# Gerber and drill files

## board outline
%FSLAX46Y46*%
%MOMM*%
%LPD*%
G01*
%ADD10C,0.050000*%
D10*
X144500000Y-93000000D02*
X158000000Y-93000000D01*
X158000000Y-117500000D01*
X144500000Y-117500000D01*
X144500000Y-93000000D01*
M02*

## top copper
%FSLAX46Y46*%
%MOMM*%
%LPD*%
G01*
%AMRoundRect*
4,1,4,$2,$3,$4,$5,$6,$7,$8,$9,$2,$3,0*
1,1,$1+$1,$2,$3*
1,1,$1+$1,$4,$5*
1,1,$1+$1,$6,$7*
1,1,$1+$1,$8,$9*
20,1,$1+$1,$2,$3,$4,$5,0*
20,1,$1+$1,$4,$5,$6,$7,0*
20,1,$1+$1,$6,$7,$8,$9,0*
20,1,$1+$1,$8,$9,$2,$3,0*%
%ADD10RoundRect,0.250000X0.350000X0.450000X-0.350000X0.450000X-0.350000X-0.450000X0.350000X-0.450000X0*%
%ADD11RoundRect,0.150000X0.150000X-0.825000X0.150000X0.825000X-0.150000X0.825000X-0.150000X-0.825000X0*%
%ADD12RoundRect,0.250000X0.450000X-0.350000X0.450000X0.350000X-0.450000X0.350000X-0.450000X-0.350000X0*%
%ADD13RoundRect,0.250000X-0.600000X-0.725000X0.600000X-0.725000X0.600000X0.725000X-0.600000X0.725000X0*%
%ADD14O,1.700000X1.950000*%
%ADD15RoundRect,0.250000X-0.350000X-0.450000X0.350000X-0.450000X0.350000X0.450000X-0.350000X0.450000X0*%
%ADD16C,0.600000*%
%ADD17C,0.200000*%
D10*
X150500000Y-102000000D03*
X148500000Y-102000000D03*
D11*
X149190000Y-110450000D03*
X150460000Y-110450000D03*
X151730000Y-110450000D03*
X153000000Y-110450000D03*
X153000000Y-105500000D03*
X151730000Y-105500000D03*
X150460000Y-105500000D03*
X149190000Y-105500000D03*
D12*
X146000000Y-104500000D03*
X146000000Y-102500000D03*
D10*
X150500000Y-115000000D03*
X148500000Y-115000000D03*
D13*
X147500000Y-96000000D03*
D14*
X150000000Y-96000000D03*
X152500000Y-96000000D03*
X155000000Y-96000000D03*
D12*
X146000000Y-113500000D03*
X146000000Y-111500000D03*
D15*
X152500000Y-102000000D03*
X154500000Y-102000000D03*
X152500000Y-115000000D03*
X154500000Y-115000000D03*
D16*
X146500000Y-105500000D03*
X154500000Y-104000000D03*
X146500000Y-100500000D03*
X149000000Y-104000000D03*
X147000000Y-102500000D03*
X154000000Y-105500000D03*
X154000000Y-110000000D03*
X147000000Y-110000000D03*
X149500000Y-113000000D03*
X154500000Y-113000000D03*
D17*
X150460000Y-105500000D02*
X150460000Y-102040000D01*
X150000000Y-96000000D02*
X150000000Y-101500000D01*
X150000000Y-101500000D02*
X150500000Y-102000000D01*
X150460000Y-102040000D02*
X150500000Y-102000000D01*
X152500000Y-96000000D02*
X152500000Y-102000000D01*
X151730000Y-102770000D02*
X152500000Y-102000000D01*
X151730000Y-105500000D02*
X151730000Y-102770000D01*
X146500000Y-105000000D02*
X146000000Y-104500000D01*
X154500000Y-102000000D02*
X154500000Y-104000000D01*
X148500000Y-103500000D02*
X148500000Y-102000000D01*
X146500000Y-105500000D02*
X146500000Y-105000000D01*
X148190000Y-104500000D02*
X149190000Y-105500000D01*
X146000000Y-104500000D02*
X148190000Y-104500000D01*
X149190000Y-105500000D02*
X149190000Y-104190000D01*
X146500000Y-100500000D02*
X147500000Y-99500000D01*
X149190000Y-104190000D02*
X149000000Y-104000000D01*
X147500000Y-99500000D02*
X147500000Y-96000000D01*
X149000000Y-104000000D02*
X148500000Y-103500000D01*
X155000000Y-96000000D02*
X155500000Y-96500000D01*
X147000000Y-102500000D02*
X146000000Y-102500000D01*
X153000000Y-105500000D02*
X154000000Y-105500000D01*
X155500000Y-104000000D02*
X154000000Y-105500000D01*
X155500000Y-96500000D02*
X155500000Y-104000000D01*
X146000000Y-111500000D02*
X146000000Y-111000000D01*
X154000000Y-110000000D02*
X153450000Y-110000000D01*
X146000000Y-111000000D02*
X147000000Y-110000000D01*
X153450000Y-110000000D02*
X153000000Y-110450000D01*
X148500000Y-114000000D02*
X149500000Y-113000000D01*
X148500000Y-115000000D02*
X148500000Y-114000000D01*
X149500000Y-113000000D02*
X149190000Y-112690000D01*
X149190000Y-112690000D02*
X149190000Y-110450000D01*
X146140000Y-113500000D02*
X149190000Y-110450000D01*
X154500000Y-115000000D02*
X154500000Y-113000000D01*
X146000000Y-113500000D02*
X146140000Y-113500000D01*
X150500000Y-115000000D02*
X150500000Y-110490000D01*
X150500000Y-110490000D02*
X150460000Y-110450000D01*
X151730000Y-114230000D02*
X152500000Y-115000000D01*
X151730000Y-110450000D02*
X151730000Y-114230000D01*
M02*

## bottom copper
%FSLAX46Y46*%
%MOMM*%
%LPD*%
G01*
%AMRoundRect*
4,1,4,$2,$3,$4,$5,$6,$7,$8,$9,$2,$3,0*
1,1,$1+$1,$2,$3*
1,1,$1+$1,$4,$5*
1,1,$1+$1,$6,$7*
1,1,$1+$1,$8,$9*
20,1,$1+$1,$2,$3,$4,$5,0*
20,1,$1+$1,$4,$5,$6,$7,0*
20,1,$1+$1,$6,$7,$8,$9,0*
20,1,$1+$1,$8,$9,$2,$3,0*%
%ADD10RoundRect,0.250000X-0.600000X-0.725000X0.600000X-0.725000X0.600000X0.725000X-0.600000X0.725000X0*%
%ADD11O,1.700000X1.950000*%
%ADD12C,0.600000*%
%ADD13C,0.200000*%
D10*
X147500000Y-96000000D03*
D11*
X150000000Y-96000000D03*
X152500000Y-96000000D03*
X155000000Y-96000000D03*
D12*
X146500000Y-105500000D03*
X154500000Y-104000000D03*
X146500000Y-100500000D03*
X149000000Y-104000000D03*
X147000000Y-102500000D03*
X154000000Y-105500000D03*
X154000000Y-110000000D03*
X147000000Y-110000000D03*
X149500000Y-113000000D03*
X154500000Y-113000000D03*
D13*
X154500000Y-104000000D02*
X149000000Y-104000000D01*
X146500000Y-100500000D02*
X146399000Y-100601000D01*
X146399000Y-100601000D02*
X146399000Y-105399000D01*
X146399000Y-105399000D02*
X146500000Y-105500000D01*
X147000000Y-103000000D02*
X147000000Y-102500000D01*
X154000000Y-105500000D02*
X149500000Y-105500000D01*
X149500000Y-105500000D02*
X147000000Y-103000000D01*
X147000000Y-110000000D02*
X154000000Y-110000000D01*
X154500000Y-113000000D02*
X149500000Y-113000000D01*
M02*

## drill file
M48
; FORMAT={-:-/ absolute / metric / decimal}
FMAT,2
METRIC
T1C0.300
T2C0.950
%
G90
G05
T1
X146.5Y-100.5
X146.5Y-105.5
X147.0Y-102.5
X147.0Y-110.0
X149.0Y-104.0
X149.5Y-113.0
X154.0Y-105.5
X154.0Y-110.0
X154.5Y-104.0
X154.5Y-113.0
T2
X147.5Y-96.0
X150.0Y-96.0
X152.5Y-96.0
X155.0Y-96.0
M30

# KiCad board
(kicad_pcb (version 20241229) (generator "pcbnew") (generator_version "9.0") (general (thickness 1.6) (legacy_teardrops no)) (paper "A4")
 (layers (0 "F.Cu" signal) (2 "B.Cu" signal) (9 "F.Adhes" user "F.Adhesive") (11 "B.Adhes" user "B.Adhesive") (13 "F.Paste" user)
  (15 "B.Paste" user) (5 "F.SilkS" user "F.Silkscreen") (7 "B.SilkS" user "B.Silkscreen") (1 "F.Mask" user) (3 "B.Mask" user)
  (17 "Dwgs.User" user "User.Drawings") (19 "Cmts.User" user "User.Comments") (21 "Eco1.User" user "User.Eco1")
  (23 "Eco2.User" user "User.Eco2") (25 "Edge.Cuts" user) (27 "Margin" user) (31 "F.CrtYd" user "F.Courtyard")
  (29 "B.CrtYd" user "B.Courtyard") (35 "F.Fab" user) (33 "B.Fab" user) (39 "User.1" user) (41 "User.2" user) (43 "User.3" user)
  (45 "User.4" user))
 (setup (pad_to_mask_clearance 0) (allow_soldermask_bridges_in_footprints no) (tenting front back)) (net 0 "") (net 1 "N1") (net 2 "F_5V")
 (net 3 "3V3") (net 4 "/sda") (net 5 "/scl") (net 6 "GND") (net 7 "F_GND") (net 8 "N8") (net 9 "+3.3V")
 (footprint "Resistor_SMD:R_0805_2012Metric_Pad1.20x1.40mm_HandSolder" (layer "F.Cu") (at 149.5 102 180)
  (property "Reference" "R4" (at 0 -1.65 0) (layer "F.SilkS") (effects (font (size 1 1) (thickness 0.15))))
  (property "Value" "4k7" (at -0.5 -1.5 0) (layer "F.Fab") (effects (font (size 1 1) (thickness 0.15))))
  (pad "1" smd roundrect (at -1 0 180) (size 1.2 1.4) (layers "F.Cu" "F.Mask" "F.Paste") (roundrect_rratio 0.208333) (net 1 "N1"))
  (pad "2" smd roundrect (at 1 0 180) (size 1.2 1.4) (layers "F.Cu" "F.Mask" "F.Paste") (roundrect_rratio 0.208333) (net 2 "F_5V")))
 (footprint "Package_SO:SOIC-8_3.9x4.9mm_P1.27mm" (layer "F.Cu") (at 151.095 107.975 90)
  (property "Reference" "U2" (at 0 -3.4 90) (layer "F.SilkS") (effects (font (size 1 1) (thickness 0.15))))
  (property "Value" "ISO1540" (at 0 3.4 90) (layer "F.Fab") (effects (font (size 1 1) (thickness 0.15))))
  (pad "1" smd roundrect (at -2.475 -1.905 90) (size 1.95 0.6) (layers "F.Cu" "F.Mask" "F.Paste") (roundrect_rratio 0.25) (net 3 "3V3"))
  (pad "2" smd roundrect (at -2.475 -0.635 90) (size 1.95 0.6) (layers "F.Cu" "F.Mask" "F.Paste") (roundrect_rratio 0.25) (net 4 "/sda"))
  (pad "3" smd roundrect (at -2.475 0.635 90) (size 1.95 0.6) (layers "F.Cu" "F.Mask" "F.Paste") (roundrect_rratio 0.25) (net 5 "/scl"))
  (pad "4" smd roundrect (at -2.475 1.905 90) (size 1.95 0.6) (layers "F.Cu" "F.Mask" "F.Paste") (roundrect_rratio 0.25) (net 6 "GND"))
  (pad "5" smd roundrect (at 2.475 1.905 90) (size 1.95 0.6) (layers "F.Cu" "F.Mask" "F.Paste") (roundrect_rratio 0.25) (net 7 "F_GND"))
  (pad "6" smd roundrect (at 2.475 0.635 90) (size 1.95 0.6) (layers "F.Cu" "F.Mask" "F.Paste") (roundrect_rratio 0.25) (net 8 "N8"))
  (pad "7" smd roundrect (at 2.475 -0.635 90) (size 1.95 0.6) (layers "F.Cu" "F.Mask" "F.Paste") (roundrect_rratio 0.25) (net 1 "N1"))
  (pad "8" smd roundrect (at 2.475 -1.905 90) (size 1.95 0.6) (layers "F.Cu" "F.Mask" "F.Paste") (roundrect_rratio 0.25) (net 2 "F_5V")))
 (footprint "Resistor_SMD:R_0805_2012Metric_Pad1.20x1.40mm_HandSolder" (layer "F.Cu") (at 146 103.5 90)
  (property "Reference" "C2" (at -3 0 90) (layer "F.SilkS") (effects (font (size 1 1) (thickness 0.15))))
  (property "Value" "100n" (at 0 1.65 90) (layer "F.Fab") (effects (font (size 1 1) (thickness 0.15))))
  (pad "1" smd roundrect (at -1 0 90) (size 1.2 1.4) (layers "F.Cu" "F.Mask" "F.Paste") (roundrect_rratio 0.208333) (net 2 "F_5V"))
  (pad "2" smd roundrect (at 1 0 90) (size 1.2 1.4) (layers "F.Cu" "F.Mask" "F.Paste") (roundrect_rratio 0.208333) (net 7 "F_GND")))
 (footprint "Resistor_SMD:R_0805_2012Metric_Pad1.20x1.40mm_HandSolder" (layer "F.Cu") (at 149.5 115 180)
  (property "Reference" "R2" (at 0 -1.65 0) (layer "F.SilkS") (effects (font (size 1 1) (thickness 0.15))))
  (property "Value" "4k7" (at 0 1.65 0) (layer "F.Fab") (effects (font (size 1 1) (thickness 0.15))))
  (pad "1" smd roundrect (at -1 0 180) (size 1.2 1.4) (layers "F.Cu" "F.Mask" "F.Paste") (roundrect_rratio 0.208333) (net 4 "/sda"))
  (pad "2" smd roundrect (at 1 0 180) (size 1.2 1.4) (layers "F.Cu" "F.Mask" "F.Paste") (roundrect_rratio 0.208333) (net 3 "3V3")))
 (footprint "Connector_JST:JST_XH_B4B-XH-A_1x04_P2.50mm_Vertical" (layer "F.Cu") (at 147.5 96)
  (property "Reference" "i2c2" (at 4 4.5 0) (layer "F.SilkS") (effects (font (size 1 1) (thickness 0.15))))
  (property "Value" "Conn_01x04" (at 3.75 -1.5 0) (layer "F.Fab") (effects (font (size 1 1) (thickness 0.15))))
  (pad "1" thru_hole roundrect (at 0 0) (size 1.7 1.95) (drill 0.95) (layers "*.Cu" "*.Mask") (remove_unused_layers no)
   (roundrect_rratio 0.147059) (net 2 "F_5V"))
  (pad "2" thru_hole oval (at 2.5 0) (size 1.7 1.95) (drill 0.95) (layers "*.Cu" "*.Mask") (remove_unused_layers no) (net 1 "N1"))
  (pad "3" thru_hole oval (at 5 0) (size 1.7 1.95) (drill 0.95) (layers "*.Cu" "*.Mask") (remove_unused_layers no) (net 8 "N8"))
  (pad "4" thru_hole oval (at 7.5 0) (size 1.7 1.95) (drill 0.95) (layers "*.Cu" "*.Mask") (remove_unused_layers no) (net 7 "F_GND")))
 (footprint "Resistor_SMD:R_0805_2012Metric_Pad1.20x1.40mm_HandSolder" (layer "F.Cu") (at 146 112.5 90)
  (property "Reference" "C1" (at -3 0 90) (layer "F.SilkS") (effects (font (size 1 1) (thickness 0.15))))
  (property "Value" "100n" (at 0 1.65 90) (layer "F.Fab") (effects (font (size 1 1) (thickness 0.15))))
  (pad "1" smd roundrect (at -1 0 90) (size 1.2 1.4) (layers "F.Cu" "F.Mask" "F.Paste") (roundrect_rratio 0.208333) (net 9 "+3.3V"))
  (pad "2" smd roundrect (at 1 0 90) (size 1.2 1.4) (layers "F.Cu" "F.Mask" "F.Paste") (roundrect_rratio 0.208333) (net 6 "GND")))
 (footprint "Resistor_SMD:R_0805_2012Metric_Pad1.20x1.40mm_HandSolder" (layer "F.Cu") (at 153.5 102)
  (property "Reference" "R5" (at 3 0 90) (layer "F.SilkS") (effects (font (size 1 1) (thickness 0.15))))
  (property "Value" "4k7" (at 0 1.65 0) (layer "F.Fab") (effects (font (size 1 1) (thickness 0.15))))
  (pad "1" smd roundrect (at -1 0) (size 1.2 1.4) (layers "F.Cu" "F.Mask" "F.Paste") (roundrect_rratio 0.208333) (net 8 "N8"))
  (pad "2" smd roundrect (at 1 0) (size 1.2 1.4) (layers "F.Cu" "F.Mask" "F.Paste") (roundrect_rratio 0.208333) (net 2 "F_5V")))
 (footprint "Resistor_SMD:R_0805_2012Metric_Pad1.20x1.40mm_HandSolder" (layer "F.Cu") (at 153.5 115)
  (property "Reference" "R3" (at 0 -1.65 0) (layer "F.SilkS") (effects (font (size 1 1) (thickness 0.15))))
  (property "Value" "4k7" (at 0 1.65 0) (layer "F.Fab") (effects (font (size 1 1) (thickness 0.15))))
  (pad "1" smd roundrect (at -1 0) (size 1.2 1.4) (layers "F.Cu" "F.Mask" "F.Paste") (roundrect_rratio 0.208333) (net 5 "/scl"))
  (pad "2" smd roundrect (at 1 0) (size 1.2 1.4) (layers "F.Cu" "F.Mask" "F.Paste") (roundrect_rratio 0.208333) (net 3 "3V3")))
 (gr_rect (start 144.5 93) (end 158 117.5) (stroke (width 0.05) (type default)) (fill no) (layer "Edge.Cuts"))
 (segment (start 150.46 105.5) (end 150.46 102.04) (width 0.2) (layer "F.Cu") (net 1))
 (segment (start 150 96) (end 150 101.5) (width 0.2) (layer "F.Cu") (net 1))
 (segment (start 150 101.5) (end 150.5 102) (width 0.2) (layer "F.Cu") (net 1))
 (segment (start 150.46 102.04) (end 150.5 102) (width 0.2) (layer "F.Cu") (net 1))
 (segment (start 152.5 96) (end 152.5 102) (width 0.2) (layer "F.Cu") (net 8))
 (segment (start 151.73 102.77) (end 152.5 102) (width 0.2) (layer "F.Cu") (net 8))
 (segment (start 151.73 105.5) (end 151.73 102.77) (width 0.2) (layer "F.Cu") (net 8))
 (segment (start 146.5 105) (end 146 104.5) (width 0.2) (layer "F.Cu") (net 2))
 (segment (start 154.5 102) (end 154.5 104) (width 0.2) (layer "F.Cu") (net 2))
 (segment (start 148.5 103.5) (end 148.5 102) (width 0.2) (layer "F.Cu") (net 2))
 (segment (start 146.5 105.5) (end 146.5 105) (width 0.2) (layer "F.Cu") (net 2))
 (segment (start 148.19 104.5) (end 149.19 105.5) (width 0.2) (layer "F.Cu") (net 2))
 (segment (start 146 104.5) (end 148.19 104.5) (width 0.2) (layer "F.Cu") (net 2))
 (segment (start 149.19 105.5) (end 149.19 104.19) (width 0.2) (layer "F.Cu") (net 2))
 (segment (start 146.5 100.5) (end 147.5 99.5) (width 0.2) (layer "F.Cu") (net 2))
 (segment (start 149.19 104.19) (end 149 104) (width 0.2) (layer "F.Cu") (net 2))
 (segment (start 147.5 99.5) (end 147.5 96) (width 0.2) (layer "F.Cu") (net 2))
 (segment (start 149 104) (end 148.5 103.5) (width 0.2) (layer "F.Cu") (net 2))
 (via (at 146.5 105.5) (size 0.6) (drill 0.3) (layers "F.Cu" "B.Cu") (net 2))
 (via (at 154.5 104) (size 0.6) (drill 0.3) (layers "F.Cu" "B.Cu") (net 2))
 (via (at 146.5 100.5) (size 0.6) (drill 0.3) (layers "F.Cu" "B.Cu") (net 2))
 (via (at 149 104) (size 0.6) (drill 0.3) (layers "F.Cu" "B.Cu") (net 2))
 (segment (start 154.5 104) (end 149 104) (width 0.2) (layer "B.Cu") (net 2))
 (segment (start 146.5 100.5) (end 146.399 100.601) (width 0.2) (layer "B.Cu") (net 2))
 (segment (start 146.399 100.601) (end 146.399 105.399) (width 0.2) (layer "B.Cu") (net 2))
 (segment (start 146.399 105.399) (end 146.5 105.5) (width 0.2) (layer "B.Cu") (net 2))
 (segment (start 155 96) (end 155.5 96.5) (width 0.2) (layer "F.Cu") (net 7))
 (segment (start 147 102.5) (end 146 102.5) (width 0.2) (layer "F.Cu") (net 7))
 (segment (start 153 105.5) (end 154 105.5) (width 0.2) (layer "F.Cu") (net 7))
 (segment (start 155.5 104) (end 154 105.5) (width 0.2) (layer "F.Cu") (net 7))
 (segment (start 155.5 96.5) (end 155.5 104) (width 0.2) (layer "F.Cu") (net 7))
 (via (at 147 102.5) (size 0.6) (drill 0.3) (layers "F.Cu" "B.Cu") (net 7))
 (via (at 154 105.5) (size 0.6) (drill 0.3) (layers "F.Cu" "B.Cu") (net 7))
 (segment (start 147 103) (end 147 102.5) (width 0.2) (layer "B.Cu") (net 7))
 (segment (start 154 105.5) (end 149.5 105.5) (width 0.2) (layer "B.Cu") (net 7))
 (segment (start 149.5 105.5) (end 147 103) (width 0.2) (layer "B.Cu") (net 7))
 (segment (start 146 111.5) (end 146 111) (width 0.2) (layer "F.Cu") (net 6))
 (segment (start 154 110) (end 153.45 110) (width 0.2) (layer "F.Cu") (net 6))
 (segment (start 146 111) (end 147 110) (width 0.2) (layer "F.Cu") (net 6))
 (segment (start 153.45 110) (end 153 110.45) (width 0.2) (layer "F.Cu") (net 6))
 (via (at 154 110) (size 0.6) (drill 0.3) (layers "F.Cu" "B.Cu") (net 6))
 (via (at 147 110) (size 0.6) (drill 0.3) (layers "F.Cu" "B.Cu") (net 6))
 (segment (start 147 110) (end 154 110) (width 0.2) (layer "B.Cu") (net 6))
 (segment (start 148.5 114) (end 149.5 113) (width 0.2) (layer "F.Cu") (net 9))
 (segment (start 148.5 115) (end 148.5 114) (width 0.2) (layer "F.Cu") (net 9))
 (segment (start 149.5 113) (end 149.19 112.69) (width 0.2) (layer "F.Cu") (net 9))
 (segment (start 149.19 112.69) (end 149.19 110.45) (width 0.2) (layer "F.Cu") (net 9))
 (segment (start 146.14 113.5) (end 149.19 110.45) (width 0.2) (layer "F.Cu") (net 9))
 (segment (start 154.5 115) (end 154.5 113) (width 0.2) (layer "F.Cu") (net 9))
 (segment (start 146 113.5) (end 146.14 113.5) (width 0.2) (layer "F.Cu") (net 9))
 (via (at 149.5 113) (size 0.6) (drill 0.3) (layers "F.Cu" "B.Cu") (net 9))
 (via (at 154.5 113) (size 0.6) (drill 0.3) (layers "F.Cu" "B.Cu") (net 9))
 (segment (start 154.5 113) (end 149.5 113) (width 0.2) (layer "B.Cu") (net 9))
 (segment (start 150.5 115) (end 150.5 110.49) (width 0.2) (layer "F.Cu") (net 4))
 (segment (start 150.5 110.49) (end 150.46 110.45) (width 0.2) (layer "F.Cu") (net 4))
 (segment (start 151.73 114.23) (end 152.5 115) (width 0.2) (layer "F.Cu") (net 5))
 (segment (start 151.73 110.45) (end 151.73 114.23) (width 0.2) (layer "F.Cu") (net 5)))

